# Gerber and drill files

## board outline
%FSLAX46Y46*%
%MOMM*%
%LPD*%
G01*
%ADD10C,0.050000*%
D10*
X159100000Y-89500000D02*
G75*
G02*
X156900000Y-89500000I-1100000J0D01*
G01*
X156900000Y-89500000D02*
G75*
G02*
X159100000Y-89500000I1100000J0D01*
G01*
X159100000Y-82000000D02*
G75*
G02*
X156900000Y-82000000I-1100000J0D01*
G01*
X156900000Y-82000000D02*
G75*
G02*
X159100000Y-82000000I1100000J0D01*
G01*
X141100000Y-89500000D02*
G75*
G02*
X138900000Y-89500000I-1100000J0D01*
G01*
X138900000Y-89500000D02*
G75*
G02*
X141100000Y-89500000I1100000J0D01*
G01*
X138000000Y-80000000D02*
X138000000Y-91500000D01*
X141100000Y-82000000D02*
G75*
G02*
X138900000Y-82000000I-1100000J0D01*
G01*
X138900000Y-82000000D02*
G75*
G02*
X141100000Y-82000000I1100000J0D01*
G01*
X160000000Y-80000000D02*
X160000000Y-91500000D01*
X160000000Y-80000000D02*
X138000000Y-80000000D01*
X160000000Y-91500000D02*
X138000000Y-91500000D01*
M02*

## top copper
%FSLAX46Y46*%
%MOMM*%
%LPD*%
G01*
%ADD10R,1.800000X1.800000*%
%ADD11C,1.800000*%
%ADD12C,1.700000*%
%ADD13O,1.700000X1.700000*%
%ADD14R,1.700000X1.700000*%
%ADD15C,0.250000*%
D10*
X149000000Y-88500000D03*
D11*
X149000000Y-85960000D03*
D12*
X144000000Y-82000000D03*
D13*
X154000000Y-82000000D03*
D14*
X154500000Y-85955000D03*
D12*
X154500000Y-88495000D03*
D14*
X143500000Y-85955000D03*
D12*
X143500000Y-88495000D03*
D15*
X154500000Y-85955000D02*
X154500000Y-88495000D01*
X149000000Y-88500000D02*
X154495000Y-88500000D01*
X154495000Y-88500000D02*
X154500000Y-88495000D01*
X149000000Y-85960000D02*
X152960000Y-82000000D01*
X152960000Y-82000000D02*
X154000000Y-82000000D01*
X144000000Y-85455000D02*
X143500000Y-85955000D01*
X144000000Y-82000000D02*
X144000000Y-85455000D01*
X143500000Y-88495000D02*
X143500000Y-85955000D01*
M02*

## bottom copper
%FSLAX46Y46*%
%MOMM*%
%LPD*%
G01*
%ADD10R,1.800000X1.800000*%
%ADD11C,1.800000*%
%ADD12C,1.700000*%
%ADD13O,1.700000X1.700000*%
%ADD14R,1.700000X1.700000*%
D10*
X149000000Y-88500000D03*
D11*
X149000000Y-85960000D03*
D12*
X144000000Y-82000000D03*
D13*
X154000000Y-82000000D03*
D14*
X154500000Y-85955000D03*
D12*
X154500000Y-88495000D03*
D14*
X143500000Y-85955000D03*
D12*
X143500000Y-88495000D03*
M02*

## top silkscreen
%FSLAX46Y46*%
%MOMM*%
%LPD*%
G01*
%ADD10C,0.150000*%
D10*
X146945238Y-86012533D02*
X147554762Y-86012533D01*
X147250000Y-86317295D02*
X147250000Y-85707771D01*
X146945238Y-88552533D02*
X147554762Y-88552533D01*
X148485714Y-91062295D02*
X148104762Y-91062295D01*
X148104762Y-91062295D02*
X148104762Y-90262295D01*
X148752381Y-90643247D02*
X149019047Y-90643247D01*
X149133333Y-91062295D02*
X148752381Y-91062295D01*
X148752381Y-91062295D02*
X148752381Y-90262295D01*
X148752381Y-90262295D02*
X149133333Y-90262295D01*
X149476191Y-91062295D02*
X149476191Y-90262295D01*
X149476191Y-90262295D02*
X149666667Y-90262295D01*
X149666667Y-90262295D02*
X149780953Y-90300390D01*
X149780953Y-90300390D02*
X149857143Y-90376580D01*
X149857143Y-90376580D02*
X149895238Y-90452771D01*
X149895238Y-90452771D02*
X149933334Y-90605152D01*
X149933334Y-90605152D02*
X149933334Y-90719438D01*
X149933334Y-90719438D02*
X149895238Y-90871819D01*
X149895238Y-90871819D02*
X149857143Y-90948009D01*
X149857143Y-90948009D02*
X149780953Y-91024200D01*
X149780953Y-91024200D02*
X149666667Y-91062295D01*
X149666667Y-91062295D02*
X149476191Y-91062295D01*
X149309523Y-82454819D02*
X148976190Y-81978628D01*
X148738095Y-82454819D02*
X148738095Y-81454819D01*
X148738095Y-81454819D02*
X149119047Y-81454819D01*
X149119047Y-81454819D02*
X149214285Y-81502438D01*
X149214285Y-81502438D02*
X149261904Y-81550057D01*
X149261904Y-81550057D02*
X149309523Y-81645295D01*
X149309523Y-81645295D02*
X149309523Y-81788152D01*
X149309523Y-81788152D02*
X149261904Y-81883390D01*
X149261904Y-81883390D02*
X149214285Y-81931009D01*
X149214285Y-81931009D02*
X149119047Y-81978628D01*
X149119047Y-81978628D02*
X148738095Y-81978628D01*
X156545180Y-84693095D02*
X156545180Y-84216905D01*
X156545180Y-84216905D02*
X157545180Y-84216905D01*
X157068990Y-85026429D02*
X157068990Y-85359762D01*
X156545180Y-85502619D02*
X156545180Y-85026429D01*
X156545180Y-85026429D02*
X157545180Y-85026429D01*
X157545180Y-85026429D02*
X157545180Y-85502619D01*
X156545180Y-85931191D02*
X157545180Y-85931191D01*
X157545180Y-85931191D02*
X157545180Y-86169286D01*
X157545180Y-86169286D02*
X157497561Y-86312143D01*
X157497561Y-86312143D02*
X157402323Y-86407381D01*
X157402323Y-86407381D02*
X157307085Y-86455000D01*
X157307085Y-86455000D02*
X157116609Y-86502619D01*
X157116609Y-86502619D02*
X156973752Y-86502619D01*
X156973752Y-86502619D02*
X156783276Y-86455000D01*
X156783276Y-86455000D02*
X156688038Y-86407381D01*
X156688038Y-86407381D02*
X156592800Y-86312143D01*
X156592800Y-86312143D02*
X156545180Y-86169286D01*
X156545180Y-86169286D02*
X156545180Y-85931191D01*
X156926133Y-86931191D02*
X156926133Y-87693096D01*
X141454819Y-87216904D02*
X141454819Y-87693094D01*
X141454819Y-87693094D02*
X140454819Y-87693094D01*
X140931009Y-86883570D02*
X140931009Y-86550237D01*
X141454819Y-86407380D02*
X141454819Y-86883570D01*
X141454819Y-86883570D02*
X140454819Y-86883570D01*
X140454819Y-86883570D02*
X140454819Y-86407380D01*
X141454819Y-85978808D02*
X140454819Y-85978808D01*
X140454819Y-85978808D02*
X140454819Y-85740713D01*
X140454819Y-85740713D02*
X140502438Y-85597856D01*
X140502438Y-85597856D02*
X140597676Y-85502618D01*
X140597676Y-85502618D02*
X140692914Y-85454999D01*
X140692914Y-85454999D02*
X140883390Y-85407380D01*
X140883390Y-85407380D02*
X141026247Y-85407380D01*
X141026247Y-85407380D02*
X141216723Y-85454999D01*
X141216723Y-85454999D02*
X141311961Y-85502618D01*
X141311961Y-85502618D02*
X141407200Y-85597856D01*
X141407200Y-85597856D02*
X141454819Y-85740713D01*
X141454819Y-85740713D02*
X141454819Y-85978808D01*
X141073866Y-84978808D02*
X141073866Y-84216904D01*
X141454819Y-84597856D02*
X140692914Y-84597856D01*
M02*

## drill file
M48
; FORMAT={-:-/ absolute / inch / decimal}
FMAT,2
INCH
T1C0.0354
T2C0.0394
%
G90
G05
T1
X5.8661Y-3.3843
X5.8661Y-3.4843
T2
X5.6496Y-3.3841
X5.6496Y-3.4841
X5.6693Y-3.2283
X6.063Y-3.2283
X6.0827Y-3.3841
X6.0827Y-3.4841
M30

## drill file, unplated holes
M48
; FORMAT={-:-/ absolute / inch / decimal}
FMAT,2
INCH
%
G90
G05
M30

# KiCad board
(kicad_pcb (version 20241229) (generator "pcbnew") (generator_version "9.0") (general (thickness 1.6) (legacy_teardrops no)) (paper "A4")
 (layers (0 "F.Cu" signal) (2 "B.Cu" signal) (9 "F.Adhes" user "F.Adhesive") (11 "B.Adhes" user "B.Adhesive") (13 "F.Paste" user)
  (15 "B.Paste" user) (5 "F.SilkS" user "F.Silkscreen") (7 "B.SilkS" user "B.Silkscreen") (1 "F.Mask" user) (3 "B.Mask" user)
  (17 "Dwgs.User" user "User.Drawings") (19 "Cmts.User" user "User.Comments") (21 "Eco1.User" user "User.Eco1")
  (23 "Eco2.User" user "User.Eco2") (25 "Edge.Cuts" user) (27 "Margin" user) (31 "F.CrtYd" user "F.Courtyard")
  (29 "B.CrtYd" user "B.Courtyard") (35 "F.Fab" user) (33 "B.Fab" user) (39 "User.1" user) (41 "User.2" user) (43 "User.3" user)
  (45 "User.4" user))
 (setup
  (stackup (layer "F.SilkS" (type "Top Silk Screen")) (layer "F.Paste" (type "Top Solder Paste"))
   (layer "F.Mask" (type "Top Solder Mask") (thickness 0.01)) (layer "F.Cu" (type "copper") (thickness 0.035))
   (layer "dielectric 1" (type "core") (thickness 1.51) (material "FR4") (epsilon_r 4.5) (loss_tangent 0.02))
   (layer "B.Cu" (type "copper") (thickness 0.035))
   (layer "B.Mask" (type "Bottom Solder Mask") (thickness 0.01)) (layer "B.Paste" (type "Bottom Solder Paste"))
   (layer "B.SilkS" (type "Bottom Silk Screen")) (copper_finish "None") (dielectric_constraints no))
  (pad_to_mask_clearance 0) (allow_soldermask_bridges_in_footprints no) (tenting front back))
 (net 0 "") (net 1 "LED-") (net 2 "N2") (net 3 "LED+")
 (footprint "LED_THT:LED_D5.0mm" (layer "F.Cu") (at 149 88.5 90)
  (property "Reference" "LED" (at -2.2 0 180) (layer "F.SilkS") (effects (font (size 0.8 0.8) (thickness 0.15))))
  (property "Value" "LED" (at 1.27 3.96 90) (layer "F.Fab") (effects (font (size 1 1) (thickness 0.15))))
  (pad "1" thru_hole rect (at 0 0 90) (size 1.8 1.8) (drill 0.9) (layers "*.Cu" "*.Mask") (remove_unused_layers no) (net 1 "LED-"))
  (pad "2" thru_hole circle (at 2.54 0 90) (size 1.8 1.8) (drill 0.9) (layers "*.Cu" "*.Mask") (remove_unused_layers no) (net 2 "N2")))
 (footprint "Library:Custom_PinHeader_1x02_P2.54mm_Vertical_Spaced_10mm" (layer "F.Cu") (at 149 82 90)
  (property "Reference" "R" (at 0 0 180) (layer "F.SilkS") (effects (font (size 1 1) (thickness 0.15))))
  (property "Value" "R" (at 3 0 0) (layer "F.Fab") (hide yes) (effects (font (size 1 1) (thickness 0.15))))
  (pad "1" thru_hole circle (at 0 -5 90) (size 1.7 1.7) (drill 1) (layers "*.Cu" "*.Mask") (remove_unused_layers no) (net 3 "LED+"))
  (pad "2" thru_hole oval (at 0 5 90) (size 1.7 1.7) (drill 1) (layers "*.Cu" "*.Mask") (remove_unused_layers no) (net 2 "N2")))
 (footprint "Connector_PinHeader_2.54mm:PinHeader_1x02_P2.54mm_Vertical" (layer "F.Cu") (at 154.5 85.955)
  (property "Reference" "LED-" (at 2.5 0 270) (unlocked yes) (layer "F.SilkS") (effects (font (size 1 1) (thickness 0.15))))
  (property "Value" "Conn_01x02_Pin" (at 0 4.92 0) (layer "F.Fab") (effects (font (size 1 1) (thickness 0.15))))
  (pad "1" thru_hole rect (at 0 0) (size 1.7 1.7) (drill 1) (layers "*.Cu" "*.Mask") (remove_unused_layers no) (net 1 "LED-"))
  (pad "2" thru_hole circle (at 0 2.54) (size 1.7 1.7) (drill 1) (layers "*.Cu" "*.Mask") (remove_unused_layers no) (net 1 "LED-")))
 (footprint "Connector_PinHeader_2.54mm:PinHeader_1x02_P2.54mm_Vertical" (layer "F.Cu") (at 143.5 85.955)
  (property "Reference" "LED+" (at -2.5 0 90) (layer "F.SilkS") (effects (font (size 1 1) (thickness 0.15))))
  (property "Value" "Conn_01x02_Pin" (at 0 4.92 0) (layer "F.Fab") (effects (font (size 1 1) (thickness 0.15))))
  (pad "1" thru_hole rect (at 0 0) (size 1.7 1.7) (drill 1) (layers "*.Cu" "*.Mask") (remove_unused_layers no) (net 3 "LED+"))
  (pad "2" thru_hole circle (at 0 2.54) (size 1.7 1.7) (drill 1) (layers "*.Cu" "*.Mask") (remove_unused_layers no) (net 3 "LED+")))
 (gr_circle (center 158 89.5) (end 159.1 89.5) (stroke (width 0.05) (type solid)) (fill no) (layer "Edge.Cuts"))
 (gr_circle (center 158 82) (end 159.1 82) (stroke (width 0.05) (type solid)) (fill no) (layer "Edge.Cuts"))
 (gr_circle (center 140 89.5) (end 141.1 89.5) (stroke (width 0.05) (type solid)) (fill no) (layer "Edge.Cuts"))
 (gr_line (start 138 80) (end 138 91.5) (stroke (width 0.05) (type solid)) (layer "Edge.Cuts"))
 (gr_circle (center 140 82) (end 141.1 82) (stroke (width 0.05) (type solid)) (fill no) (layer "Edge.Cuts"))
 (gr_line (start 160 80) (end 160 91.5) (stroke (width 0.05) (type solid)) (layer "Edge.Cuts"))
 (gr_line (start 160 80) (end 138 80) (stroke (width 0.05) (type solid)) (layer "Edge.Cuts"))
 (gr_line (start 160 91.5) (end 138 91.5) (stroke (width 0.05) (type solid)) (layer "Edge.Cuts"))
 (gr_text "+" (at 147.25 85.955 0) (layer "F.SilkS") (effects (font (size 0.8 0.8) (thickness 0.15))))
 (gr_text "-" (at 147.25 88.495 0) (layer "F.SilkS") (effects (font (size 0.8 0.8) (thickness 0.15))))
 (segment (start 154.5 85.955) (end 154.5 88.495) (width 0.25) (layer "F.Cu") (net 1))
 (segment (start 149 88.5) (end 154.495 88.5) (width 0.25) (layer "F.Cu") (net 1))
 (segment (start 154.495 88.5) (end 154.5 88.495) (width 0.25) (layer "F.Cu") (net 1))
 (segment (start 149 85.96) (end 152.96 82) (width 0.25) (layer "F.Cu") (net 2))
 (segment (start 152.96 82) (end 154 82) (width 0.25) (layer "F.Cu") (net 2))
 (segment (start 144 85.455) (end 143.5 85.955) (width 0.25) (layer "F.Cu") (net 3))
 (segment (start 144 82) (end 144 85.455) (width 0.25) (layer "F.Cu") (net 3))
 (segment (start 143.5 88.495) (end 143.5 85.955) (width 0.25) (layer "F.Cu") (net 3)))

